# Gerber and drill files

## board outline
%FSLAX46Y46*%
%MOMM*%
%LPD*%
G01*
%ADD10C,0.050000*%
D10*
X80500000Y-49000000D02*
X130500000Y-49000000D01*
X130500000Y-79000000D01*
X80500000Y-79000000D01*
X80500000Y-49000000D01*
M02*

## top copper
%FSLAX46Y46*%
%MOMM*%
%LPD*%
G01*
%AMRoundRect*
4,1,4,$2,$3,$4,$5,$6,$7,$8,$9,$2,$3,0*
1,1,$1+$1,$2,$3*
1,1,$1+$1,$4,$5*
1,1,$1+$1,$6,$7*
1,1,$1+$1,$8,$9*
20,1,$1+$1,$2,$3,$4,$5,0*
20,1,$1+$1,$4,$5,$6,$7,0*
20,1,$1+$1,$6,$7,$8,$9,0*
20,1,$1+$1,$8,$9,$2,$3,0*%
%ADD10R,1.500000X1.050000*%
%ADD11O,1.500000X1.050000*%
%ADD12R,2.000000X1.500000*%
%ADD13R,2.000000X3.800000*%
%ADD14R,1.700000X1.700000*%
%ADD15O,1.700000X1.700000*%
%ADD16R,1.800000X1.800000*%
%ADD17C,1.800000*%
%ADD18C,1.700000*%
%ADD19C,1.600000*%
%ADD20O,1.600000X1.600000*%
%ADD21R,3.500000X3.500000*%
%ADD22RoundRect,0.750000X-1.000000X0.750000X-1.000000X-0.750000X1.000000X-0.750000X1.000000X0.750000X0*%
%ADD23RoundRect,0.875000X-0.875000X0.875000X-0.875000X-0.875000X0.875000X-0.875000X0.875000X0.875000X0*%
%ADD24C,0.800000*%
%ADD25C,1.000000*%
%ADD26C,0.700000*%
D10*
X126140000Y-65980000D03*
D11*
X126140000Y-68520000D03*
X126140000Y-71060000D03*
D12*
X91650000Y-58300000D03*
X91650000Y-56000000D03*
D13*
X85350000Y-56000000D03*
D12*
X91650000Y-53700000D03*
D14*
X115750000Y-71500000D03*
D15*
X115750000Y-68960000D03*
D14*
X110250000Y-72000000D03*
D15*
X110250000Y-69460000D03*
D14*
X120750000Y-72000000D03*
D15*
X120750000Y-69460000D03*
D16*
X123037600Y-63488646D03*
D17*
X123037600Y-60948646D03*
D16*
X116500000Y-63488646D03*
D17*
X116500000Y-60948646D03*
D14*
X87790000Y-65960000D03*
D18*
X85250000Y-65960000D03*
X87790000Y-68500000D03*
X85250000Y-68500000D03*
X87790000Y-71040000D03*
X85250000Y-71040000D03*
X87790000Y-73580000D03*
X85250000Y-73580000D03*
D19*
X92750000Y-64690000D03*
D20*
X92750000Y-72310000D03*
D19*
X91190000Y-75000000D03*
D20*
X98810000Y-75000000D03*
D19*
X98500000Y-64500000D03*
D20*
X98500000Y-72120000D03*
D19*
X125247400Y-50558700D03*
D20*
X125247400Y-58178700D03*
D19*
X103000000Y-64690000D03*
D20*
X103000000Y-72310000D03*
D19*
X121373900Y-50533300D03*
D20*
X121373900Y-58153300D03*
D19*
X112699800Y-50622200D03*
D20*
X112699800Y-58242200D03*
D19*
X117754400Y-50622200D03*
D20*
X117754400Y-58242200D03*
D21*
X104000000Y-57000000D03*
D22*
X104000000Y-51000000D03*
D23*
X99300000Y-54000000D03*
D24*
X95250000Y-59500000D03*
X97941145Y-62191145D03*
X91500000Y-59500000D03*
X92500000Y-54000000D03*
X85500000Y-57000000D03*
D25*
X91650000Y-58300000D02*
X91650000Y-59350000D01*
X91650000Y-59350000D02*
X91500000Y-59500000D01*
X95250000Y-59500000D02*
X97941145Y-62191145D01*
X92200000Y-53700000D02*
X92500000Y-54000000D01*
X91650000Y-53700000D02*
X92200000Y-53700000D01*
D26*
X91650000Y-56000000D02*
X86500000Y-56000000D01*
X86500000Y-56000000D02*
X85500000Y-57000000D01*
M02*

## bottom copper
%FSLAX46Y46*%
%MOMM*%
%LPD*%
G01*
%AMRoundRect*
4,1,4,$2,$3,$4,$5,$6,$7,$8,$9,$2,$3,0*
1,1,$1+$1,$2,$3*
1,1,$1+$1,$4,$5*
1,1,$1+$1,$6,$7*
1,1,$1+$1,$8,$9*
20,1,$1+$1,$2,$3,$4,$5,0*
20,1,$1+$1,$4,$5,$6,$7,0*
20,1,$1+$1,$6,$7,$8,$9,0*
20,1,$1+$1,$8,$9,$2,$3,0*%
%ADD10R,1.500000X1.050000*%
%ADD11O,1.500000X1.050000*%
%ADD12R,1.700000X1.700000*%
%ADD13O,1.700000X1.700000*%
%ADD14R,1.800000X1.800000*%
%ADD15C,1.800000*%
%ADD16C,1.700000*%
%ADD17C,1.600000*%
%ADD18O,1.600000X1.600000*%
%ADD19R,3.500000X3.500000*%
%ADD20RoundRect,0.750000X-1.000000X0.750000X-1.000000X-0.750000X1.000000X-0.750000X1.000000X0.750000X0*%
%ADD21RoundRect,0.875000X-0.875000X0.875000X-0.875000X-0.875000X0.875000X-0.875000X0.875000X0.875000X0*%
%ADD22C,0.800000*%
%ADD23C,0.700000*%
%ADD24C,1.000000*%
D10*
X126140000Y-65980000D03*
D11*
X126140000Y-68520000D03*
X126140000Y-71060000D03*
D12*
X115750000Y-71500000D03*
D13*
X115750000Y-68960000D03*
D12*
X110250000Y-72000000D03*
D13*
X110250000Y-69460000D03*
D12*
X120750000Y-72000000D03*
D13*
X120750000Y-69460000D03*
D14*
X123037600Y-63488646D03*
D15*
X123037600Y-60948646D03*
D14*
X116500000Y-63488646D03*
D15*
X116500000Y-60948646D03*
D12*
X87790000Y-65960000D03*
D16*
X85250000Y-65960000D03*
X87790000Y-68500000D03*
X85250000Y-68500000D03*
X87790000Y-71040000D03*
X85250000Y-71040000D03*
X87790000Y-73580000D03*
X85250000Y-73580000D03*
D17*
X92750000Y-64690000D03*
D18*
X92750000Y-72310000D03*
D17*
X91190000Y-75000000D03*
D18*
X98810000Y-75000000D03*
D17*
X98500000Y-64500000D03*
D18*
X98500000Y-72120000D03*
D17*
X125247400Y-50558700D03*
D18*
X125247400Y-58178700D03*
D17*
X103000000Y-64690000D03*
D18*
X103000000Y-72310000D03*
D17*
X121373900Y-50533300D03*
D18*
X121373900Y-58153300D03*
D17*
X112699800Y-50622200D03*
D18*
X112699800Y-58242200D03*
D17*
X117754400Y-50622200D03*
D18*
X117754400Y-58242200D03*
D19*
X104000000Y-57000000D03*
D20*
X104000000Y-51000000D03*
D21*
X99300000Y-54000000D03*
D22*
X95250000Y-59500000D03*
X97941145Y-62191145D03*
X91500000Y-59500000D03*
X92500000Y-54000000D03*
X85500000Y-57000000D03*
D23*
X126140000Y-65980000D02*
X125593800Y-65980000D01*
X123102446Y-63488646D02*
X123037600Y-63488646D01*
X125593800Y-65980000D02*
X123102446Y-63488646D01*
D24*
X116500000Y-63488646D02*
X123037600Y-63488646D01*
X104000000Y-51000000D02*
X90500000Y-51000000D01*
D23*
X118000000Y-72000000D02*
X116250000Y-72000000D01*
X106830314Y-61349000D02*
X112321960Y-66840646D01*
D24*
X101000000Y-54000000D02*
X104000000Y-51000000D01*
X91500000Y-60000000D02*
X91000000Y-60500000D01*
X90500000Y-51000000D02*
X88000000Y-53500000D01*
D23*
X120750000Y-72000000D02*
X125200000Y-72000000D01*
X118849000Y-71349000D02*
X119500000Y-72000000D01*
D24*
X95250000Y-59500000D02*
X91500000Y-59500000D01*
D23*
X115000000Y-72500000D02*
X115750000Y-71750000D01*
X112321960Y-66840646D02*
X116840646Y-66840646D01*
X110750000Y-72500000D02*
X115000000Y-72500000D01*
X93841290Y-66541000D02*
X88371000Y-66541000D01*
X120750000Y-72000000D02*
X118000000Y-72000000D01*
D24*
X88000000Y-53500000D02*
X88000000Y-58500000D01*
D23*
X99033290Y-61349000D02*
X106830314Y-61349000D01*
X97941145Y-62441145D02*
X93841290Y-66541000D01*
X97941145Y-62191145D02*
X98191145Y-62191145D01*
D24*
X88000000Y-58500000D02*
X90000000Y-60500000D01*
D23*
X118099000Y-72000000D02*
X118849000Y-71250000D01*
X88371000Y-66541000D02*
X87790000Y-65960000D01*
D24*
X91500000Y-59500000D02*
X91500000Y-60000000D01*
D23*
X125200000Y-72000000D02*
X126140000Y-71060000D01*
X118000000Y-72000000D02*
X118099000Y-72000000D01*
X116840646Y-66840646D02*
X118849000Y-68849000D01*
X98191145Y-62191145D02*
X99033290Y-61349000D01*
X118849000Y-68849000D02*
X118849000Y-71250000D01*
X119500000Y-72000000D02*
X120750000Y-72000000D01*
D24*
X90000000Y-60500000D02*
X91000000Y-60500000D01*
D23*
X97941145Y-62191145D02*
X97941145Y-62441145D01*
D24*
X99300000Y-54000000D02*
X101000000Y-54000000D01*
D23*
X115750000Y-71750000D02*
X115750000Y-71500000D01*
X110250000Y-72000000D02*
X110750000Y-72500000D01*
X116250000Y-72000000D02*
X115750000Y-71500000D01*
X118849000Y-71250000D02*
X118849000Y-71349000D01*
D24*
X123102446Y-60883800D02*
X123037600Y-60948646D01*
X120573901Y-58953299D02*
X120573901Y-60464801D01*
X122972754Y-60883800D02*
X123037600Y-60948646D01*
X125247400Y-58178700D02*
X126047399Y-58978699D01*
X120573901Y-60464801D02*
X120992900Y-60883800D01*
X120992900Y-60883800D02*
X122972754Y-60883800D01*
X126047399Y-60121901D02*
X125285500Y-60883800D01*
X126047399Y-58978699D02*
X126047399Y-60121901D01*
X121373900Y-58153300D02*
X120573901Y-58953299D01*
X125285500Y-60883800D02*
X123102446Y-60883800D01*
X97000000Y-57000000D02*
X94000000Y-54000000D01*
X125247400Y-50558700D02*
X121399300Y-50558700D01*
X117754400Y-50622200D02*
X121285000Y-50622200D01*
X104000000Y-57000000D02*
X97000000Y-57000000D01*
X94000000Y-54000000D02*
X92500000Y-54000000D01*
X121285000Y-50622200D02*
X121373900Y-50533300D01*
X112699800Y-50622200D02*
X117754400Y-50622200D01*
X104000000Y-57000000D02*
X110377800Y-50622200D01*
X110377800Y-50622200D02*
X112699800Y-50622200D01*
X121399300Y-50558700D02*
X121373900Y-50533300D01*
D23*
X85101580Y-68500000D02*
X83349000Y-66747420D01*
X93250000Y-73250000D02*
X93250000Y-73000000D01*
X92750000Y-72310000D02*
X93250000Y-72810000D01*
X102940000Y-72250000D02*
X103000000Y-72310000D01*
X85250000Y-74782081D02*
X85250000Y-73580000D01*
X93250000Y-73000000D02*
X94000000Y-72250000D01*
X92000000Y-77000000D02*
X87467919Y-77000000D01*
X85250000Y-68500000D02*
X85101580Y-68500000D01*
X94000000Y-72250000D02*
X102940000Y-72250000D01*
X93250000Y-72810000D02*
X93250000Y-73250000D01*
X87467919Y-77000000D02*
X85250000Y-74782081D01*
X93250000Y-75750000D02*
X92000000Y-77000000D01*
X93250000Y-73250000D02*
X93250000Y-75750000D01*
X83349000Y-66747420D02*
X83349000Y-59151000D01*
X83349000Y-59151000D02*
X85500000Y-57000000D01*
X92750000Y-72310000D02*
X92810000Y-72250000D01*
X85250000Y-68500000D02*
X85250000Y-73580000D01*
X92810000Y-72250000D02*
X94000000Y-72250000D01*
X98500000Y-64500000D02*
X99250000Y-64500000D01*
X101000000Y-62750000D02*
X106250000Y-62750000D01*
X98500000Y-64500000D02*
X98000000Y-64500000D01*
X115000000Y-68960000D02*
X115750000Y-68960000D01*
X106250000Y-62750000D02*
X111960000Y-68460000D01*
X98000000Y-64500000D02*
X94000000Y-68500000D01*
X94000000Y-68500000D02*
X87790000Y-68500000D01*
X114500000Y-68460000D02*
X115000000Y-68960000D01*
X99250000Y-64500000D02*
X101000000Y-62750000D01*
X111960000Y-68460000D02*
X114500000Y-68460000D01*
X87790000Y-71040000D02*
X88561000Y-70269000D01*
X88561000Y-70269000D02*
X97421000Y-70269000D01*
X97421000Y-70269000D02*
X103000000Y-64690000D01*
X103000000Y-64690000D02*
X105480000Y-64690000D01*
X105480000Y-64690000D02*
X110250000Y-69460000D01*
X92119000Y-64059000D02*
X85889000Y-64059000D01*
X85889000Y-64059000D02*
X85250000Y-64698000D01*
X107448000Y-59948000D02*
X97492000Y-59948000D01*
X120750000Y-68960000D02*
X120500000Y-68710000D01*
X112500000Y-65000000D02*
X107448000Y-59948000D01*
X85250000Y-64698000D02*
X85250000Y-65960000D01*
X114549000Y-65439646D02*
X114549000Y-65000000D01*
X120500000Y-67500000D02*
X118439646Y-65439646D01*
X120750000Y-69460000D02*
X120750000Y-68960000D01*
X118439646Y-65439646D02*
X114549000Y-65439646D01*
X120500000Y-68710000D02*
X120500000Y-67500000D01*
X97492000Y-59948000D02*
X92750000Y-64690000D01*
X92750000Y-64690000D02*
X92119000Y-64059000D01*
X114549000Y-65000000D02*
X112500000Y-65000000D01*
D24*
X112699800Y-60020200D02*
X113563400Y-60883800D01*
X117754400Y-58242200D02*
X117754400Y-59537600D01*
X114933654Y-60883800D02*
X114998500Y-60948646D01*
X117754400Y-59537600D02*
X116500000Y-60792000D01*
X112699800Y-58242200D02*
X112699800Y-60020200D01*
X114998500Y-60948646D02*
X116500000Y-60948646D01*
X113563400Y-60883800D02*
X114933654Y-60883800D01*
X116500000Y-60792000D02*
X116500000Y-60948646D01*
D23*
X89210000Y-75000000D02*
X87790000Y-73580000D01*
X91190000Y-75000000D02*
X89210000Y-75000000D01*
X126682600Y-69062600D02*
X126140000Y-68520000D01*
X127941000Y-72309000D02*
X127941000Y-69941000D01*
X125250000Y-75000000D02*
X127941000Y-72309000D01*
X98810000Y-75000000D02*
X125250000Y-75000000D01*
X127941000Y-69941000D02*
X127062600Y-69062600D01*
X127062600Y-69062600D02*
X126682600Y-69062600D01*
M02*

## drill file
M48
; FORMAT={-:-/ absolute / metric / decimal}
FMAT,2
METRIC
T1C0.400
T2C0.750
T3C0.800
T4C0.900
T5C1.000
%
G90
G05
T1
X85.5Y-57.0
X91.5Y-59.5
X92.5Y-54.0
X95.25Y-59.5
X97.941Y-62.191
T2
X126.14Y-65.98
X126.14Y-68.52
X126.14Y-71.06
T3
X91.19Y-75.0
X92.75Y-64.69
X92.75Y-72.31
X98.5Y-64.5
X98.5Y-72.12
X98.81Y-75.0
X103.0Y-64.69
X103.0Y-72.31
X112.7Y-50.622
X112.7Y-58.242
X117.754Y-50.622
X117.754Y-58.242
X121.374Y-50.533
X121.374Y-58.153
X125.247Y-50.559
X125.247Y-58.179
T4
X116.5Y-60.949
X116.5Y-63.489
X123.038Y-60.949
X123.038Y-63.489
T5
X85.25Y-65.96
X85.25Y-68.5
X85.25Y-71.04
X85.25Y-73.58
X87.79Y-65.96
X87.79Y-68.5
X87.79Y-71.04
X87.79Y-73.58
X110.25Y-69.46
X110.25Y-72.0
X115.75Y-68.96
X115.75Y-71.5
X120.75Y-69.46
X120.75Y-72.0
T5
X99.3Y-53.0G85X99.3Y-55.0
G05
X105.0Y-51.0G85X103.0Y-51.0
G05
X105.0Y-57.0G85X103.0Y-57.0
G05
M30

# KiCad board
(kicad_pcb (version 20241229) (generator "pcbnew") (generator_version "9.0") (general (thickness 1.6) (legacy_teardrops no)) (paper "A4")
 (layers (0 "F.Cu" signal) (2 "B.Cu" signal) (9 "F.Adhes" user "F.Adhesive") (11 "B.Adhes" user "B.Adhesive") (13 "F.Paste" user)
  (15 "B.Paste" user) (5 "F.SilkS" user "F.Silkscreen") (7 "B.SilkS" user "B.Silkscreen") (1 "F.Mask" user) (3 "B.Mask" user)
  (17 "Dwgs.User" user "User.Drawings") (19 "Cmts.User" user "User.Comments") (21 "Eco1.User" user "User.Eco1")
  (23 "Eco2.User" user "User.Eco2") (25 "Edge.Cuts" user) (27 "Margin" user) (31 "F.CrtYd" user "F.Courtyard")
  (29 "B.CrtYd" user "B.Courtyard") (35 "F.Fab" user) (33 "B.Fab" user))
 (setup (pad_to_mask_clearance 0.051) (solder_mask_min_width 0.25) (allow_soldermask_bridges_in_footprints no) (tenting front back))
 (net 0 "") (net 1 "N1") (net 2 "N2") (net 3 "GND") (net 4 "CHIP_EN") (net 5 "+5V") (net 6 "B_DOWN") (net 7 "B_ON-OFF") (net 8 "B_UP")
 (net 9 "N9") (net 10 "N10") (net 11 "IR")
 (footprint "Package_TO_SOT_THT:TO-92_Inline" (layer "F.Cu") (at 126.14 67.25 -90)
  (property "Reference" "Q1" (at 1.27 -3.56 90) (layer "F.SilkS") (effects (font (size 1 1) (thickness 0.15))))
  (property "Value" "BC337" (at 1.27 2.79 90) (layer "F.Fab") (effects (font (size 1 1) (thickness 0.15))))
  (pad "1" thru_hole rect (at -1.27 0 270) (size 1.05 1.5) (drill 0.75) (layers "*.Cu" "*.Mask") (remove_unused_layers no) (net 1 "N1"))
  (pad "2" thru_hole oval (at 1.27 0 270) (size 1.05 1.5) (drill 0.75) (layers "*.Cu" "*.Mask") (remove_unused_layers no) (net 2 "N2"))
  (pad "3" thru_hole oval (at 3.81 0 270) (size 1.05 1.5) (drill 0.75) (layers "*.Cu" "*.Mask") (remove_unused_layers no) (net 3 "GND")))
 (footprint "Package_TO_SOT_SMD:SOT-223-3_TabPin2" (layer "F.Cu") (at 88.5 56 180)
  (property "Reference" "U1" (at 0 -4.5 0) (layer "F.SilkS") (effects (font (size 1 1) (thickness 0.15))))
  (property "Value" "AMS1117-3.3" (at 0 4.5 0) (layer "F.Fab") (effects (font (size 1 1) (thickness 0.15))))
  (pad "1" smd rect (at -3.15 -2.3 180) (size 2 1.5) (layers "F.Cu" "F.Mask" "F.Paste") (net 3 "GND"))
  (pad "2" smd rect (at -3.15 0 180) (size 2 1.5) (layers "F.Cu" "F.Mask" "F.Paste") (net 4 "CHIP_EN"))
  (pad "2" smd rect (at 3.15 0 180) (size 2 3.8) (layers "F.Cu" "F.Mask" "F.Paste") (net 4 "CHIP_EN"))
  (pad "3" smd rect (at -3.15 2.3 180) (size 2 1.5) (layers "F.Cu" "F.Mask" "F.Paste") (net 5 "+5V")))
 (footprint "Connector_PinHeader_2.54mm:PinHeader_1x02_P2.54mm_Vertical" (layer "F.Cu") (at 115.75 71.5 180)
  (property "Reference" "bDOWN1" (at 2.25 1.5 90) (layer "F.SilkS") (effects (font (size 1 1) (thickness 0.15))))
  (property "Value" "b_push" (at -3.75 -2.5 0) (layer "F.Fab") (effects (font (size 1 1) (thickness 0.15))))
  (pad "1" thru_hole rect (at 0 0 180) (size 1.7 1.7) (drill 1) (layers "*.Cu" "*.Mask") (remove_unused_layers no) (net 3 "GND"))
  (pad "2" thru_hole oval (at 0 2.54 180) (size 1.7 1.7) (drill 1) (layers "*.Cu" "*.Mask") (remove_unused_layers no) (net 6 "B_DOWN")))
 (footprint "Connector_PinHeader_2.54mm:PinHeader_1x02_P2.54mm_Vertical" (layer "F.Cu") (at 110.25 72 180)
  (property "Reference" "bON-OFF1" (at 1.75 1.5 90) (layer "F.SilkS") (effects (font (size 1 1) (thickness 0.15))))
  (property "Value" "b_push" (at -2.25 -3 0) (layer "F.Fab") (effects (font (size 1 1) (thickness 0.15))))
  (pad "1" thru_hole rect (at 0 0 180) (size 1.7 1.7) (drill 1) (layers "*.Cu" "*.Mask") (remove_unused_layers no) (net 3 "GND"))
  (pad "2" thru_hole oval (at 0 2.54 180) (size 1.7 1.7) (drill 1) (layers "*.Cu" "*.Mask") (remove_unused_layers no) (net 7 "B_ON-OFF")))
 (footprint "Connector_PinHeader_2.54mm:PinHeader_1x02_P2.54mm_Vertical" (layer "F.Cu") (at 120.75 72 180)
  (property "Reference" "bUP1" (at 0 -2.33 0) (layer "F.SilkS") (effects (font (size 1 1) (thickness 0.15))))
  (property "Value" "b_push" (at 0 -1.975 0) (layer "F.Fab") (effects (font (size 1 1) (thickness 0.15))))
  (pad "1" thru_hole rect (at 0 0 180) (size 1.7 1.7) (drill 1) (layers "*.Cu" "*.Mask") (remove_unused_layers no) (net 3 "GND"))
  (pad "2" thru_hole oval (at 0 2.54 180) (size 1.7 1.7) (drill 1) (layers "*.Cu" "*.Mask") (remove_unused_layers no) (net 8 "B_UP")))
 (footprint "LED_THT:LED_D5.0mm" (layer "F.Cu") (at 123.0376 63.488646 90)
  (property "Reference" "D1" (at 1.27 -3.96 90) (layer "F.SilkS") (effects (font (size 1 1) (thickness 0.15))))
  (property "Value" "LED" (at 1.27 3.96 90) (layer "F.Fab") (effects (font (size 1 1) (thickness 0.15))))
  (pad "1" thru_hole rect (at 0 0 90) (size 1.8 1.8) (drill 0.9) (layers "*.Cu" "*.Mask") (remove_unused_layers no) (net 1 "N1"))
  (pad "2" thru_hole circle (at 2.54 0 90) (size 1.8 1.8) (drill 0.9) (layers "*.Cu" "*.Mask") (remove_unused_layers no) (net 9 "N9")))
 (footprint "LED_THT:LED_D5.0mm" (layer "F.Cu") (at 116.5 63.488646 90)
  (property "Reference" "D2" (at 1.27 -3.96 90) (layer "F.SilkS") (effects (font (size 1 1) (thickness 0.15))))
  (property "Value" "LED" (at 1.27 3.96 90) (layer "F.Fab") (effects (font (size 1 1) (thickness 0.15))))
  (pad "1" thru_hole rect (at 0 0 90) (size 1.8 1.8) (drill 0.9) (layers "*.Cu" "*.Mask") (remove_unused_layers no) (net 1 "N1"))
  (pad "2" thru_hole circle (at 2.54 0 90) (size 1.8 1.8) (drill 0.9) (layers "*.Cu" "*.Mask") (remove_unused_layers no) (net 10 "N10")))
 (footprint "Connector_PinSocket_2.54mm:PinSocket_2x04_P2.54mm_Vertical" (layer "F.Cu") (at 87.79 65.96)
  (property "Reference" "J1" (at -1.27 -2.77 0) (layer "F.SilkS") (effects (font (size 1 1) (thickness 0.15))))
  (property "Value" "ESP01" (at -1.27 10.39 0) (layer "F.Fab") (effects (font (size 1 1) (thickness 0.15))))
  (pad "1" thru_hole rect (at 0 0) (size 1.7 1.7) (drill 1) (layers "*.Cu" "*.Mask") (remove_unused_layers no) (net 3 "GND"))
  (pad "2" thru_hole circle (at -2.54 0) (size 1.7 1.7) (drill 1) (layers "*.Cu" "*.Mask") (remove_unused_layers no) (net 8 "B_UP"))
  (pad "3" thru_hole circle (at 0 2.54) (size 1.7 1.7) (drill 1) (layers "*.Cu" "*.Mask") (remove_unused_layers no) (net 6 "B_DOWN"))
  (pad "4" thru_hole circle (at -2.54 2.54) (size 1.7 1.7) (drill 1) (layers "*.Cu" "*.Mask") (remove_unused_layers no) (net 4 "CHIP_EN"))
  (pad "5" thru_hole circle (at 0 5.08) (size 1.7 1.7) (drill 1) (layers "*.Cu" "*.Mask") (remove_unused_layers no) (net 7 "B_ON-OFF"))
  (pad "6" thru_hole circle (at -2.54 5.08) (size 1.7 1.7) (drill 1) (layers "*.Cu" "*.Mask") (remove_unused_layers no) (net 4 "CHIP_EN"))
  (pad "7" thru_hole circle (at 0 7.62) (size 1.7 1.7) (drill 1) (layers "*.Cu" "*.Mask") (remove_unused_layers no) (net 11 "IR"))
  (pad "8" thru_hole circle (at -2.54 7.62) (size 1.7 1.7) (drill 1) (layers "*.Cu" "*.Mask") (remove_unused_layers no) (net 4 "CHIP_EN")))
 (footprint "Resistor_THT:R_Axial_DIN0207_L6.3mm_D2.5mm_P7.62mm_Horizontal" (layer "F.Cu") (at 92.75 64.69 -90)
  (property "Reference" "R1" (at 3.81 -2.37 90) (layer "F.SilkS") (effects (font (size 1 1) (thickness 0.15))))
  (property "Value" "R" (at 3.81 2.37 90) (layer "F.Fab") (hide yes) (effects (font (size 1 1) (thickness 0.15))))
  (pad "1" thru_hole circle (at 0 0 270) (size 1.6 1.6) (drill 0.8) (layers "*.Cu" "*.Mask") (remove_unused_layers no) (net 8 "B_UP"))
  (pad "2" thru_hole oval (at 7.62 0 270) (size 1.6 1.6) (drill 0.8) (layers "*.Cu" "*.Mask") (remove_unused_layers no) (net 4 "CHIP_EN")))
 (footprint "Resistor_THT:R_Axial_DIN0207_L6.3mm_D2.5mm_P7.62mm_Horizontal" (layer "F.Cu") (at 91.19 75)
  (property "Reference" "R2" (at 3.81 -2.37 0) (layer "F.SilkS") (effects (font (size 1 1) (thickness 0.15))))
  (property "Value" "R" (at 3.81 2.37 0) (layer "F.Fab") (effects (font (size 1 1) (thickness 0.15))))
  (pad "1" thru_hole circle (at 0 0) (size 1.6 1.6) (drill 0.8) (layers "*.Cu" "*.Mask") (remove_unused_layers no) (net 11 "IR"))
  (pad "2" thru_hole oval (at 7.62 0) (size 1.6 1.6) (drill 0.8) (layers "*.Cu" "*.Mask") (remove_unused_layers no) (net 2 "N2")))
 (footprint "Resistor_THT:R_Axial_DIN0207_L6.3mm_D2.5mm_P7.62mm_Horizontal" (layer "F.Cu") (at 98.5 64.5 -90)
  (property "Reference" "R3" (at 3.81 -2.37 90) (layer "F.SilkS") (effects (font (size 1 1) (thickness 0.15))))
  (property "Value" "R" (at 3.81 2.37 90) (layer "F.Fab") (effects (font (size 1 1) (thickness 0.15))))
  (pad "1" thru_hole circle (at 0 0 270) (size 1.6 1.6) (drill 0.8) (layers "*.Cu" "*.Mask") (remove_unused_layers no) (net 6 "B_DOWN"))
  (pad "2" thru_hole oval (at 7.62 0 270) (size 1.6 1.6) (drill 0.8) (layers "*.Cu" "*.Mask") (remove_unused_layers no) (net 4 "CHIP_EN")))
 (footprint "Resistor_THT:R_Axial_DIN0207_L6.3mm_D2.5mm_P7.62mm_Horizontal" (layer "F.Cu") (at 125.2474 50.5587 -90)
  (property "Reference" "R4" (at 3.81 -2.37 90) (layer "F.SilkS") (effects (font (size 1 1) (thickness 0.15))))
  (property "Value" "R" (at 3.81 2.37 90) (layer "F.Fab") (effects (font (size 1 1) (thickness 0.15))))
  (pad "1" thru_hole circle (at 0 0 270) (size 1.6 1.6) (drill 0.8) (layers "*.Cu" "*.Mask") (remove_unused_layers no) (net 5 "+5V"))
  (pad "2" thru_hole oval (at 7.62 0 270) (size 1.6 1.6) (drill 0.8) (layers "*.Cu" "*.Mask") (remove_unused_layers no) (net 9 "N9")))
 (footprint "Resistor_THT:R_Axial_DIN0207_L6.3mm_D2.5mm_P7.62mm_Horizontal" (layer "F.Cu") (at 103 64.69 -90)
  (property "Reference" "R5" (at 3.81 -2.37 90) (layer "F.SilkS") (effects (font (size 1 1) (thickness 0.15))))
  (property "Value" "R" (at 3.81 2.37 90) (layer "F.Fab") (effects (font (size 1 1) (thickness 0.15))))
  (pad "1" thru_hole circle (at 0 0 270) (size 1.6 1.6) (drill 0.8) (layers "*.Cu" "*.Mask") (remove_unused_layers no) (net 7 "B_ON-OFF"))
  (pad "2" thru_hole oval (at 7.62 0 270) (size 1.6 1.6) (drill 0.8) (layers "*.Cu" "*.Mask") (remove_unused_layers no) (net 4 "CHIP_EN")))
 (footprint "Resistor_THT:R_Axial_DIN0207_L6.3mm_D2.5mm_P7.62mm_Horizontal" (layer "F.Cu") (at 121.3739 50.5333 -90)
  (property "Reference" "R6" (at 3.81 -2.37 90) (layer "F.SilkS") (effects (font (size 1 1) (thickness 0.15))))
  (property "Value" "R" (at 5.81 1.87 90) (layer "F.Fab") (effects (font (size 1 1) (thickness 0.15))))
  (pad "1" thru_hole circle (at 0 0 270) (size 1.6 1.6) (drill 0.8) (layers "*.Cu" "*.Mask") (remove_unused_layers no) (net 5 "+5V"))
  (pad "2" thru_hole oval (at 7.62 0 270) (size 1.6 1.6) (drill 0.8) (layers "*.Cu" "*.Mask") (remove_unused_layers no) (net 9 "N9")))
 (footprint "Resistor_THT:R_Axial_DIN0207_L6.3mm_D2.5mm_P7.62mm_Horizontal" (layer "F.Cu") (at 112.6998 50.6222 -90)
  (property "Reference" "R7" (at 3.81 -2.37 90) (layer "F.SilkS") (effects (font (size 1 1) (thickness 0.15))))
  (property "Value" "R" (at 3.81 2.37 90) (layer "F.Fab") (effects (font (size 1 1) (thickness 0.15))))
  (pad "1" thru_hole circle (at 0 0 270) (size 1.6 1.6) (drill 0.8) (layers "*.Cu" "*.Mask") (remove_unused_layers no) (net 5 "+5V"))
  (pad "2" thru_hole oval (at 7.62 0 270) (size 1.6 1.6) (drill 0.8) (layers "*.Cu" "*.Mask") (remove_unused_layers no) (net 10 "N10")))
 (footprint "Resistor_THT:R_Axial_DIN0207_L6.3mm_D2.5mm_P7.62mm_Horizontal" (layer "F.Cu") (at 117.7544 50.6222 -90)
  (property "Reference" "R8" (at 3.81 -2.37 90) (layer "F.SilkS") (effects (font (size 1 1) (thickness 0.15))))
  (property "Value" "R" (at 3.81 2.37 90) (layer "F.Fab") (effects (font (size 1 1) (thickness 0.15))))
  (pad "1" thru_hole circle (at 0 0 270) (size 1.6 1.6) (drill 0.8) (layers "*.Cu" "*.Mask") (remove_unused_layers no) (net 5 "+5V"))
  (pad "2" thru_hole oval (at 7.62 0 270) (size 1.6 1.6) (drill 0.8) (layers "*.Cu" "*.Mask") (remove_unused_layers no) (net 10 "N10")))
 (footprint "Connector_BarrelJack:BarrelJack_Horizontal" (layer "F.Cu") (at 104 57 -90)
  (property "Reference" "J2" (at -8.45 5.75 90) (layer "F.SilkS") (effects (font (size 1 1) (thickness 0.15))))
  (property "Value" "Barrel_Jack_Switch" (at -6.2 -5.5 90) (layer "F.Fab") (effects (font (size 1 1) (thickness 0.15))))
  (pad "1" thru_hole rect (at 0 0 270) (size 3.5 3.5) (drill oval 1 3) (layers "*.Cu" "*.Mask") (remove_unused_layers no) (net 5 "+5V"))
  (pad "2" thru_hole roundrect (at -6 0 270) (size 3 3.5) (drill oval 1 3) (layers "*.Cu" "*.Mask") (remove_unused_layers no)
   (roundrect_rratio 0.25) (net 3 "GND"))
  (pad "3" thru_hole roundrect (at -3 4.7 270) (size 3.5 3.5) (drill oval 3 1) (layers "*.Cu" "*.Mask") (remove_unused_layers no)
   (roundrect_rratio 0.25) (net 3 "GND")))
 (gr_rect (start 80.5 49) (end 130.5 79) (stroke (width 0.05) (type solid)) (fill no) (layer "Edge.Cuts"))
 (segment (start 126.14 65.98) (end 125.5938 65.98) (width 0.7) (layer "B.Cu") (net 1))
 (segment (start 123.102446 63.488646) (end 123.0376 63.488646) (width 0.7) (layer "B.Cu") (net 1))
 (segment (start 125.5938 65.98) (end 123.102446 63.488646) (width 0.7) (layer "B.Cu") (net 1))
 (segment (start 116.5 63.488646) (end 123.0376 63.488646) (width 1) (layer "B.Cu") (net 1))
 (segment (start 91.65 58.3) (end 91.65 59.35) (width 1) (layer "F.Cu") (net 3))
 (segment (start 91.65 59.35) (end 91.5 59.5) (width 1) (layer "F.Cu") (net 3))
 (segment (start 95.25 59.5) (end 97.941145 62.191145) (width 1) (layer "F.Cu") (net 3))
 (via (at 95.25 59.5) (size 0.8) (drill 0.4) (layers "F.Cu" "B.Cu") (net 3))
 (via (at 97.941145 62.191145) (size 0.8) (drill 0.4) (layers "F.Cu" "B.Cu") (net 3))
 (via (at 91.5 59.5) (size 0.8) (drill 0.4) (layers "F.Cu" "B.Cu") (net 3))
 (segment (start 104 51) (end 90.5 51) (width 1) (layer "B.Cu") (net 3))
 (segment (start 118 72) (end 116.25 72) (width 0.7) (layer "B.Cu") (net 3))
 (segment (start 106.830314 61.349) (end 112.32196 66.840646) (width 0.7) (layer "B.Cu") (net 3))
 (segment (start 101 54) (end 104 51) (width 1) (layer "B.Cu") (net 3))
 (segment (start 91.5 60) (end 91 60.5) (width 1) (layer "B.Cu") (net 3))
 (segment (start 90.5 51) (end 88 53.5) (width 1) (layer "B.Cu") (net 3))
 (segment (start 120.75 72) (end 125.2 72) (width 0.7) (layer "B.Cu") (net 3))
 (segment (start 118.849 71.349) (end 119.5 72) (width 0.7) (layer "B.Cu") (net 3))
 (segment (start 95.25 59.5) (end 91.5 59.5) (width 1) (layer "B.Cu") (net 3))
 (segment (start 115 72.5) (end 115.75 71.75) (width 0.7) (layer "B.Cu") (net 3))
 (segment (start 112.32196 66.840646) (end 116.840646 66.840646) (width 0.7) (layer "B.Cu") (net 3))
 (segment (start 110.75 72.5) (end 115 72.5) (width 0.7) (layer "B.Cu") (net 3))
 (segment (start 93.84129 66.541) (end 88.371 66.541) (width 0.7) (layer "B.Cu") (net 3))
 (segment (start 120.75 72) (end 118 72) (width 0.7) (layer "B.Cu") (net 3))
 (segment (start 88 53.5) (end 88 58.5) (width 1) (layer "B.Cu") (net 3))
 (segment (start 99.03329 61.349) (end 106.830314 61.349) (width 0.7) (layer "B.Cu") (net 3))
 (segment (start 97.941145 62.441145) (end 93.84129 66.541) (width 0.7) (layer "B.Cu") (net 3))
 (segment (start 97.941145 62.191145) (end 98.191145 62.191145) (width 0.7) (layer "B.Cu") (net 3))
 (segment (start 88 58.5) (end 90 60.5) (width 1) (layer "B.Cu") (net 3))
 (segment (start 118.099 72) (end 118.849 71.25) (width 0.7) (layer "B.Cu") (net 3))
 (segment (start 88.371 66.541) (end 87.79 65.96) (width 0.7) (layer "B.Cu") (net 3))
 (segment (start 91.5 59.5) (end 91.5 60) (width 1) (layer "B.Cu") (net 3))
 (segment (start 125.2 72) (end 126.14 71.06) (width 0.7) (layer "B.Cu") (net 3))
 (segment (start 118 72) (end 118.099 72) (width 0.7) (layer "B.Cu") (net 3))
 (segment (start 116.840646 66.840646) (end 118.849 68.849) (width 0.7) (layer "B.Cu") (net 3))
 (segment (start 98.191145 62.191145) (end 99.03329 61.349) (width 0.7) (layer "B.Cu") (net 3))
 (segment (start 118.849 68.849) (end 118.849 71.25) (width 0.7) (layer "B.Cu") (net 3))
 (segment (start 119.5 72) (end 120.75 72) (width 0.7) (layer "B.Cu") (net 3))
 (segment (start 90 60.5) (end 91 60.5) (width 1) (layer "B.Cu") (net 3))
 (segment (start 97.941145 62.191145) (end 97.941145 62.441145) (width 0.7) (layer "B.Cu") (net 3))
 (segment (start 99.3 54) (end 101 54) (width 1) (layer "B.Cu") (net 3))
 (segment (start 115.75 71.75) (end 115.75 71.5) (width 0.7) (layer "B.Cu") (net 3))
 (segment (start 110.25 72) (end 110.75 72.5) (width 0.7) (layer "B.Cu") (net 3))
 (segment (start 116.25 72) (end 115.75 71.5) (width 0.7) (layer "B.Cu") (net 3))
 (segment (start 118.849 71.25) (end 118.849 71.349) (width 0.7) (layer "B.Cu") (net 3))
 (segment (start 123.102446 60.8838) (end 123.0376 60.948646) (width 1) (layer "B.Cu") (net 9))
 (segment (start 120.573901 58.953299) (end 120.573901 60.464801) (width 1) (layer "B.Cu") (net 9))
 (segment (start 122.972754 60.8838) (end 123.0376 60.948646) (width 1) (layer "B.Cu") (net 9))
 (segment (start 125.2474 58.1787) (end 126.047399 58.978699) (width 1) (layer "B.Cu") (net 9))
 (segment (start 120.573901 60.464801) (end 120.9929 60.8838) (width 1) (layer "B.Cu") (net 9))
 (segment (start 120.9929 60.8838) (end 122.972754 60.8838) (width 1) (layer "B.Cu") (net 9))
 (segment (start 126.047399 60.121901) (end 125.2855 60.8838) (width 1) (layer "B.Cu") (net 9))
 (segment (start 126.047399 58.978699) (end 126.047399 60.121901) (width 1) (layer "B.Cu") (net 9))
 (segment (start 121.3739 58.1533) (end 120.573901 58.953299) (width 1) (layer "B.Cu") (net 9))
 (segment (start 125.2855 60.8838) (end 123.102446 60.8838) (width 1) (layer "B.Cu") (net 9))
 (segment (start 92.2 53.7) (end 92.5 54) (width 1) (layer "F.Cu") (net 5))
 (segment (start 91.65 53.7) (end 92.2 53.7) (width 1) (layer "F.Cu") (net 5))
 (via (at 92.5 54) (size 0.8) (drill 0.4) (layers "F.Cu" "B.Cu") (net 5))
 (segment (start 97 57) (end 94 54) (width 1) (layer "B.Cu") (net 5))
 (segment (start 125.2474 50.5587) (end 121.3993 50.5587) (width 1) (layer "B.Cu") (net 5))
 (segment (start 117.7544 50.6222) (end 121.285 50.6222) (width 1) (layer "B.Cu") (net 5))
 (segment (start 104 57) (end 97 57) (width 1) (layer "B.Cu") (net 5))
 (segment (start 94 54) (end 92.5 54) (width 1) (layer "B.Cu") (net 5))
 (segment (start 121.285 50.6222) (end 121.3739 50.5333) (width 1) (layer "B.Cu") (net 5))
 (segment (start 112.6998 50.6222) (end 117.7544 50.6222) (width 1) (layer "B.Cu") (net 5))
 (segment (start 104 57) (end 110.3778 50.6222) (width 1) (layer "B.Cu") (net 5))
 (segment (start 110.3778 50.6222) (end 112.6998 50.6222) (width 1) (layer "B.Cu") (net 5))
 (segment (start 121.3993 50.5587) (end 121.3739 50.5333) (width 1) (layer "B.Cu") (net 5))
 (segment (start 91.65 56) (end 86.5 56) (width 0.7) (layer "F.Cu") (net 4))
 (segment (start 86.5 56) (end 85.5 57) (width 0.7) (layer "F.Cu") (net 4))
 (via (at 85.5 57) (size 0.8) (drill 0.4) (layers "F.Cu" "B.Cu") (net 4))
 (segment (start 85.10158 68.5) (end 83.349 66.74742) (width 0.7) (layer "B.Cu") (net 4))
 (segment (start 93.25 73.25) (end 93.25 73) (width 0.7) (layer "B.Cu") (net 4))
 (segment (start 92.75 72.31) (end 93.25 72.81) (width 0.7) (layer "B.Cu") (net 4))
 (segment (start 102.94 72.25) (end 103 72.31) (width 0.7) (layer "B.Cu") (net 4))
 (segment (start 85.25 74.782081) (end 85.25 73.58) (width 0.7) (layer "B.Cu") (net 4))
 (segment (start 93.25 73) (end 94 72.25) (width 0.7) (layer "B.Cu") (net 4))
 (segment (start 92 77) (end 87.467919 77) (width 0.7) (layer "B.Cu") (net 4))
 (segment (start 85.25 68.5) (end 85.10158 68.5) (width 0.7) (layer "B.Cu") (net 4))
 (segment (start 94 72.25) (end 102.94 72.25) (width 0.7) (layer "B.Cu") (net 4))
 (segment (start 93.25 72.81) (end 93.25 73.25) (width 0.7) (layer "B.Cu") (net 4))
 (segment (start 87.467919 77) (end 85.25 74.782081) (width 0.7) (layer "B.Cu") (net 4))
 (segment (start 93.25 75.75) (end 92 77) (width 0.7) (layer "B.Cu") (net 4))
 (segment (start 93.25 73.25) (end 93.25 75.75) (width 0.7) (layer "B.Cu") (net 4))
 (segment (start 83.349 66.74742) (end 83.349 59.151) (width 0.7) (layer "B.Cu") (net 4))
 (segment (start 83.349 59.151) (end 85.5 57) (width 0.7) (layer "B.Cu") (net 4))
 (segment (start 92.75 72.31) (end 92.81 72.25) (width 0.7) (layer "B.Cu") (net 4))
 (segment (start 85.25 68.5) (end 85.25 73.58) (width 0.7) (layer "B.Cu") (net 4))
 (segment (start 92.81 72.25) (end 94 72.25) (width 0.7) (layer "B.Cu") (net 4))
 (segment (start 98.5 64.5) (end 99.25 64.5) (width 0.7) (layer "B.Cu") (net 6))
 (segment (start 101 62.75) (end 106.25 62.75) (width 0.7) (layer "B.Cu") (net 6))
 (segment (start 98.5 64.5) (end 98 64.5) (width 0.7) (layer "B.Cu") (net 6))
 (segment (start 115 68.96) (end 115.75 68.96) (width 0.7) (layer "B.Cu") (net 6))
 (segment (start 106.25 62.75) (end 111.96 68.46) (width 0.7) (layer "B.Cu") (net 6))
 (segment (start 98 64.5) (end 94 68.5) (width 0.7) (layer "B.Cu") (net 6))
 (segment (start 94 68.5) (end 87.79 68.5) (width 0.7) (layer "B.Cu") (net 6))
 (segment (start 114.5 68.46) (end 115 68.96) (width 0.7) (layer "B.Cu") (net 6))
 (segment (start 99.25 64.5) (end 101 62.75) (width 0.7) (layer "B.Cu") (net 6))
 (segment (start 111.96 68.46) (end 114.5 68.46) (width 0.7) (layer "B.Cu") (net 6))
 (segment (start 87.79 71.04) (end 88.561 70.269) (width 0.7) (layer "B.Cu") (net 7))
 (segment (start 88.561 70.269) (end 97.421 70.269) (width 0.7) (layer "B.Cu") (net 7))
 (segment (start 97.421 70.269) (end 103 64.69) (width 0.7) (layer "B.Cu") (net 7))
 (segment (start 103 64.69) (end 105.48 64.69) (width 0.7) (layer "B.Cu") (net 7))
 (segment (start 105.48 64.69) (end 110.25 69.46) (width 0.7) (layer "B.Cu") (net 7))
 (segment (start 92.119 64.059) (end 85.889 64.059) (width 0.7) (layer "B.Cu") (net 8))
 (segment (start 85.889 64.059) (end 85.25 64.698) (width 0.7) (layer "B.Cu") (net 8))
 (segment (start 107.448 59.948) (end 97.492 59.948) (width 0.7) (layer "B.Cu") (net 8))
 (segment (start 120.75 68.96) (end 120.5 68.71) (width 0.7) (layer "B.Cu") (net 8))
 (segment (start 112.5 65) (end 107.448 59.948) (width 0.7) (layer "B.Cu") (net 8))
 (segment (start 85.25 64.698) (end 85.25 65.96) (width 0.7) (layer "B.Cu") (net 8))
 (segment (start 114.549 65.439646) (end 114.549 65) (width 0.7) (layer "B.Cu") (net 8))
 (segment (start 120.5 67.5) (end 118.439646 65.439646) (width 0.7) (layer "B.Cu") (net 8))
 (segment (start 120.75 69.46) (end 120.75 68.96) (width 0.7) (layer "B.Cu") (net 8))
 (segment (start 118.439646 65.439646) (end 114.549 65.439646) (width 0.7) (layer "B.Cu") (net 8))
 (segment (start 120.5 68.71) (end 120.5 67.5) (width 0.7) (layer "B.Cu") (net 8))
 (segment (start 97.492 59.948) (end 92.75 64.69) (width 0.7) (layer "B.Cu") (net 8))
 (segment (start 92.75 64.69) (end 92.119 64.059) (width 0.7) (layer "B.Cu") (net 8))
 (segment (start 114.549 65) (end 112.5 65) (width 0.7) (layer "B.Cu") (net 8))
 (segment (start 112.6998 60.0202) (end 113.5634 60.8838) (width 1) (layer "B.Cu") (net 10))
 (segment (start 117.7544 58.2422) (end 117.7544 59.5376) (width 1) (layer "B.Cu") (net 10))
 (segment (start 114.933654 60.8838) (end 114.9985 60.948646) (width 1) (layer "B.Cu") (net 10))
 (segment (start 117.7544 59.5376) (end 116.5 60.792) (width 1) (layer "B.Cu") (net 10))
 (segment (start 112.6998 58.2422) (end 112.6998 60.0202) (width 1) (layer "B.Cu") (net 10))
 (segment (start 114.9985 60.948646) (end 116.5 60.948646) (width 1) (layer "B.Cu") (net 10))
 (segment (start 113.5634 60.8838) (end 114.933654 60.8838) (width 1) (layer "B.Cu") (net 10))
 (segment (start 116.5 60.792) (end 116.5 60.948646) (width 1) (layer "B.Cu") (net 10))
 (segment (start 89.21 75) (end 87.79 73.58) (width 0.7) (layer "B.Cu") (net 11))
 (segment (start 91.19 75) (end 89.21 75) (width 0.7) (layer "B.Cu") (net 11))
 (segment (start 126.6826 69.0626) (end 126.14 68.52) (width 0.7) (layer "B.Cu") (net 2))
 (segment (start 127.941 72.309) (end 127.941 69.941) (width 0.7) (layer "B.Cu") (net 2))
 (segment (start 125.25 75) (end 127.941 72.309) (width 0.7) (layer "B.Cu") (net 2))
 (segment (start 98.81 75) (end 125.25 75) (width 0.7) (layer "B.Cu") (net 2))
 (segment (start 127.941 69.941) (end 127.0626 69.0626) (width 0.7) (layer "B.Cu") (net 2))
 (segment (start 127.0626 69.0626) (end 126.6826 69.0626) (width 0.7) (layer "B.Cu") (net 2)))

